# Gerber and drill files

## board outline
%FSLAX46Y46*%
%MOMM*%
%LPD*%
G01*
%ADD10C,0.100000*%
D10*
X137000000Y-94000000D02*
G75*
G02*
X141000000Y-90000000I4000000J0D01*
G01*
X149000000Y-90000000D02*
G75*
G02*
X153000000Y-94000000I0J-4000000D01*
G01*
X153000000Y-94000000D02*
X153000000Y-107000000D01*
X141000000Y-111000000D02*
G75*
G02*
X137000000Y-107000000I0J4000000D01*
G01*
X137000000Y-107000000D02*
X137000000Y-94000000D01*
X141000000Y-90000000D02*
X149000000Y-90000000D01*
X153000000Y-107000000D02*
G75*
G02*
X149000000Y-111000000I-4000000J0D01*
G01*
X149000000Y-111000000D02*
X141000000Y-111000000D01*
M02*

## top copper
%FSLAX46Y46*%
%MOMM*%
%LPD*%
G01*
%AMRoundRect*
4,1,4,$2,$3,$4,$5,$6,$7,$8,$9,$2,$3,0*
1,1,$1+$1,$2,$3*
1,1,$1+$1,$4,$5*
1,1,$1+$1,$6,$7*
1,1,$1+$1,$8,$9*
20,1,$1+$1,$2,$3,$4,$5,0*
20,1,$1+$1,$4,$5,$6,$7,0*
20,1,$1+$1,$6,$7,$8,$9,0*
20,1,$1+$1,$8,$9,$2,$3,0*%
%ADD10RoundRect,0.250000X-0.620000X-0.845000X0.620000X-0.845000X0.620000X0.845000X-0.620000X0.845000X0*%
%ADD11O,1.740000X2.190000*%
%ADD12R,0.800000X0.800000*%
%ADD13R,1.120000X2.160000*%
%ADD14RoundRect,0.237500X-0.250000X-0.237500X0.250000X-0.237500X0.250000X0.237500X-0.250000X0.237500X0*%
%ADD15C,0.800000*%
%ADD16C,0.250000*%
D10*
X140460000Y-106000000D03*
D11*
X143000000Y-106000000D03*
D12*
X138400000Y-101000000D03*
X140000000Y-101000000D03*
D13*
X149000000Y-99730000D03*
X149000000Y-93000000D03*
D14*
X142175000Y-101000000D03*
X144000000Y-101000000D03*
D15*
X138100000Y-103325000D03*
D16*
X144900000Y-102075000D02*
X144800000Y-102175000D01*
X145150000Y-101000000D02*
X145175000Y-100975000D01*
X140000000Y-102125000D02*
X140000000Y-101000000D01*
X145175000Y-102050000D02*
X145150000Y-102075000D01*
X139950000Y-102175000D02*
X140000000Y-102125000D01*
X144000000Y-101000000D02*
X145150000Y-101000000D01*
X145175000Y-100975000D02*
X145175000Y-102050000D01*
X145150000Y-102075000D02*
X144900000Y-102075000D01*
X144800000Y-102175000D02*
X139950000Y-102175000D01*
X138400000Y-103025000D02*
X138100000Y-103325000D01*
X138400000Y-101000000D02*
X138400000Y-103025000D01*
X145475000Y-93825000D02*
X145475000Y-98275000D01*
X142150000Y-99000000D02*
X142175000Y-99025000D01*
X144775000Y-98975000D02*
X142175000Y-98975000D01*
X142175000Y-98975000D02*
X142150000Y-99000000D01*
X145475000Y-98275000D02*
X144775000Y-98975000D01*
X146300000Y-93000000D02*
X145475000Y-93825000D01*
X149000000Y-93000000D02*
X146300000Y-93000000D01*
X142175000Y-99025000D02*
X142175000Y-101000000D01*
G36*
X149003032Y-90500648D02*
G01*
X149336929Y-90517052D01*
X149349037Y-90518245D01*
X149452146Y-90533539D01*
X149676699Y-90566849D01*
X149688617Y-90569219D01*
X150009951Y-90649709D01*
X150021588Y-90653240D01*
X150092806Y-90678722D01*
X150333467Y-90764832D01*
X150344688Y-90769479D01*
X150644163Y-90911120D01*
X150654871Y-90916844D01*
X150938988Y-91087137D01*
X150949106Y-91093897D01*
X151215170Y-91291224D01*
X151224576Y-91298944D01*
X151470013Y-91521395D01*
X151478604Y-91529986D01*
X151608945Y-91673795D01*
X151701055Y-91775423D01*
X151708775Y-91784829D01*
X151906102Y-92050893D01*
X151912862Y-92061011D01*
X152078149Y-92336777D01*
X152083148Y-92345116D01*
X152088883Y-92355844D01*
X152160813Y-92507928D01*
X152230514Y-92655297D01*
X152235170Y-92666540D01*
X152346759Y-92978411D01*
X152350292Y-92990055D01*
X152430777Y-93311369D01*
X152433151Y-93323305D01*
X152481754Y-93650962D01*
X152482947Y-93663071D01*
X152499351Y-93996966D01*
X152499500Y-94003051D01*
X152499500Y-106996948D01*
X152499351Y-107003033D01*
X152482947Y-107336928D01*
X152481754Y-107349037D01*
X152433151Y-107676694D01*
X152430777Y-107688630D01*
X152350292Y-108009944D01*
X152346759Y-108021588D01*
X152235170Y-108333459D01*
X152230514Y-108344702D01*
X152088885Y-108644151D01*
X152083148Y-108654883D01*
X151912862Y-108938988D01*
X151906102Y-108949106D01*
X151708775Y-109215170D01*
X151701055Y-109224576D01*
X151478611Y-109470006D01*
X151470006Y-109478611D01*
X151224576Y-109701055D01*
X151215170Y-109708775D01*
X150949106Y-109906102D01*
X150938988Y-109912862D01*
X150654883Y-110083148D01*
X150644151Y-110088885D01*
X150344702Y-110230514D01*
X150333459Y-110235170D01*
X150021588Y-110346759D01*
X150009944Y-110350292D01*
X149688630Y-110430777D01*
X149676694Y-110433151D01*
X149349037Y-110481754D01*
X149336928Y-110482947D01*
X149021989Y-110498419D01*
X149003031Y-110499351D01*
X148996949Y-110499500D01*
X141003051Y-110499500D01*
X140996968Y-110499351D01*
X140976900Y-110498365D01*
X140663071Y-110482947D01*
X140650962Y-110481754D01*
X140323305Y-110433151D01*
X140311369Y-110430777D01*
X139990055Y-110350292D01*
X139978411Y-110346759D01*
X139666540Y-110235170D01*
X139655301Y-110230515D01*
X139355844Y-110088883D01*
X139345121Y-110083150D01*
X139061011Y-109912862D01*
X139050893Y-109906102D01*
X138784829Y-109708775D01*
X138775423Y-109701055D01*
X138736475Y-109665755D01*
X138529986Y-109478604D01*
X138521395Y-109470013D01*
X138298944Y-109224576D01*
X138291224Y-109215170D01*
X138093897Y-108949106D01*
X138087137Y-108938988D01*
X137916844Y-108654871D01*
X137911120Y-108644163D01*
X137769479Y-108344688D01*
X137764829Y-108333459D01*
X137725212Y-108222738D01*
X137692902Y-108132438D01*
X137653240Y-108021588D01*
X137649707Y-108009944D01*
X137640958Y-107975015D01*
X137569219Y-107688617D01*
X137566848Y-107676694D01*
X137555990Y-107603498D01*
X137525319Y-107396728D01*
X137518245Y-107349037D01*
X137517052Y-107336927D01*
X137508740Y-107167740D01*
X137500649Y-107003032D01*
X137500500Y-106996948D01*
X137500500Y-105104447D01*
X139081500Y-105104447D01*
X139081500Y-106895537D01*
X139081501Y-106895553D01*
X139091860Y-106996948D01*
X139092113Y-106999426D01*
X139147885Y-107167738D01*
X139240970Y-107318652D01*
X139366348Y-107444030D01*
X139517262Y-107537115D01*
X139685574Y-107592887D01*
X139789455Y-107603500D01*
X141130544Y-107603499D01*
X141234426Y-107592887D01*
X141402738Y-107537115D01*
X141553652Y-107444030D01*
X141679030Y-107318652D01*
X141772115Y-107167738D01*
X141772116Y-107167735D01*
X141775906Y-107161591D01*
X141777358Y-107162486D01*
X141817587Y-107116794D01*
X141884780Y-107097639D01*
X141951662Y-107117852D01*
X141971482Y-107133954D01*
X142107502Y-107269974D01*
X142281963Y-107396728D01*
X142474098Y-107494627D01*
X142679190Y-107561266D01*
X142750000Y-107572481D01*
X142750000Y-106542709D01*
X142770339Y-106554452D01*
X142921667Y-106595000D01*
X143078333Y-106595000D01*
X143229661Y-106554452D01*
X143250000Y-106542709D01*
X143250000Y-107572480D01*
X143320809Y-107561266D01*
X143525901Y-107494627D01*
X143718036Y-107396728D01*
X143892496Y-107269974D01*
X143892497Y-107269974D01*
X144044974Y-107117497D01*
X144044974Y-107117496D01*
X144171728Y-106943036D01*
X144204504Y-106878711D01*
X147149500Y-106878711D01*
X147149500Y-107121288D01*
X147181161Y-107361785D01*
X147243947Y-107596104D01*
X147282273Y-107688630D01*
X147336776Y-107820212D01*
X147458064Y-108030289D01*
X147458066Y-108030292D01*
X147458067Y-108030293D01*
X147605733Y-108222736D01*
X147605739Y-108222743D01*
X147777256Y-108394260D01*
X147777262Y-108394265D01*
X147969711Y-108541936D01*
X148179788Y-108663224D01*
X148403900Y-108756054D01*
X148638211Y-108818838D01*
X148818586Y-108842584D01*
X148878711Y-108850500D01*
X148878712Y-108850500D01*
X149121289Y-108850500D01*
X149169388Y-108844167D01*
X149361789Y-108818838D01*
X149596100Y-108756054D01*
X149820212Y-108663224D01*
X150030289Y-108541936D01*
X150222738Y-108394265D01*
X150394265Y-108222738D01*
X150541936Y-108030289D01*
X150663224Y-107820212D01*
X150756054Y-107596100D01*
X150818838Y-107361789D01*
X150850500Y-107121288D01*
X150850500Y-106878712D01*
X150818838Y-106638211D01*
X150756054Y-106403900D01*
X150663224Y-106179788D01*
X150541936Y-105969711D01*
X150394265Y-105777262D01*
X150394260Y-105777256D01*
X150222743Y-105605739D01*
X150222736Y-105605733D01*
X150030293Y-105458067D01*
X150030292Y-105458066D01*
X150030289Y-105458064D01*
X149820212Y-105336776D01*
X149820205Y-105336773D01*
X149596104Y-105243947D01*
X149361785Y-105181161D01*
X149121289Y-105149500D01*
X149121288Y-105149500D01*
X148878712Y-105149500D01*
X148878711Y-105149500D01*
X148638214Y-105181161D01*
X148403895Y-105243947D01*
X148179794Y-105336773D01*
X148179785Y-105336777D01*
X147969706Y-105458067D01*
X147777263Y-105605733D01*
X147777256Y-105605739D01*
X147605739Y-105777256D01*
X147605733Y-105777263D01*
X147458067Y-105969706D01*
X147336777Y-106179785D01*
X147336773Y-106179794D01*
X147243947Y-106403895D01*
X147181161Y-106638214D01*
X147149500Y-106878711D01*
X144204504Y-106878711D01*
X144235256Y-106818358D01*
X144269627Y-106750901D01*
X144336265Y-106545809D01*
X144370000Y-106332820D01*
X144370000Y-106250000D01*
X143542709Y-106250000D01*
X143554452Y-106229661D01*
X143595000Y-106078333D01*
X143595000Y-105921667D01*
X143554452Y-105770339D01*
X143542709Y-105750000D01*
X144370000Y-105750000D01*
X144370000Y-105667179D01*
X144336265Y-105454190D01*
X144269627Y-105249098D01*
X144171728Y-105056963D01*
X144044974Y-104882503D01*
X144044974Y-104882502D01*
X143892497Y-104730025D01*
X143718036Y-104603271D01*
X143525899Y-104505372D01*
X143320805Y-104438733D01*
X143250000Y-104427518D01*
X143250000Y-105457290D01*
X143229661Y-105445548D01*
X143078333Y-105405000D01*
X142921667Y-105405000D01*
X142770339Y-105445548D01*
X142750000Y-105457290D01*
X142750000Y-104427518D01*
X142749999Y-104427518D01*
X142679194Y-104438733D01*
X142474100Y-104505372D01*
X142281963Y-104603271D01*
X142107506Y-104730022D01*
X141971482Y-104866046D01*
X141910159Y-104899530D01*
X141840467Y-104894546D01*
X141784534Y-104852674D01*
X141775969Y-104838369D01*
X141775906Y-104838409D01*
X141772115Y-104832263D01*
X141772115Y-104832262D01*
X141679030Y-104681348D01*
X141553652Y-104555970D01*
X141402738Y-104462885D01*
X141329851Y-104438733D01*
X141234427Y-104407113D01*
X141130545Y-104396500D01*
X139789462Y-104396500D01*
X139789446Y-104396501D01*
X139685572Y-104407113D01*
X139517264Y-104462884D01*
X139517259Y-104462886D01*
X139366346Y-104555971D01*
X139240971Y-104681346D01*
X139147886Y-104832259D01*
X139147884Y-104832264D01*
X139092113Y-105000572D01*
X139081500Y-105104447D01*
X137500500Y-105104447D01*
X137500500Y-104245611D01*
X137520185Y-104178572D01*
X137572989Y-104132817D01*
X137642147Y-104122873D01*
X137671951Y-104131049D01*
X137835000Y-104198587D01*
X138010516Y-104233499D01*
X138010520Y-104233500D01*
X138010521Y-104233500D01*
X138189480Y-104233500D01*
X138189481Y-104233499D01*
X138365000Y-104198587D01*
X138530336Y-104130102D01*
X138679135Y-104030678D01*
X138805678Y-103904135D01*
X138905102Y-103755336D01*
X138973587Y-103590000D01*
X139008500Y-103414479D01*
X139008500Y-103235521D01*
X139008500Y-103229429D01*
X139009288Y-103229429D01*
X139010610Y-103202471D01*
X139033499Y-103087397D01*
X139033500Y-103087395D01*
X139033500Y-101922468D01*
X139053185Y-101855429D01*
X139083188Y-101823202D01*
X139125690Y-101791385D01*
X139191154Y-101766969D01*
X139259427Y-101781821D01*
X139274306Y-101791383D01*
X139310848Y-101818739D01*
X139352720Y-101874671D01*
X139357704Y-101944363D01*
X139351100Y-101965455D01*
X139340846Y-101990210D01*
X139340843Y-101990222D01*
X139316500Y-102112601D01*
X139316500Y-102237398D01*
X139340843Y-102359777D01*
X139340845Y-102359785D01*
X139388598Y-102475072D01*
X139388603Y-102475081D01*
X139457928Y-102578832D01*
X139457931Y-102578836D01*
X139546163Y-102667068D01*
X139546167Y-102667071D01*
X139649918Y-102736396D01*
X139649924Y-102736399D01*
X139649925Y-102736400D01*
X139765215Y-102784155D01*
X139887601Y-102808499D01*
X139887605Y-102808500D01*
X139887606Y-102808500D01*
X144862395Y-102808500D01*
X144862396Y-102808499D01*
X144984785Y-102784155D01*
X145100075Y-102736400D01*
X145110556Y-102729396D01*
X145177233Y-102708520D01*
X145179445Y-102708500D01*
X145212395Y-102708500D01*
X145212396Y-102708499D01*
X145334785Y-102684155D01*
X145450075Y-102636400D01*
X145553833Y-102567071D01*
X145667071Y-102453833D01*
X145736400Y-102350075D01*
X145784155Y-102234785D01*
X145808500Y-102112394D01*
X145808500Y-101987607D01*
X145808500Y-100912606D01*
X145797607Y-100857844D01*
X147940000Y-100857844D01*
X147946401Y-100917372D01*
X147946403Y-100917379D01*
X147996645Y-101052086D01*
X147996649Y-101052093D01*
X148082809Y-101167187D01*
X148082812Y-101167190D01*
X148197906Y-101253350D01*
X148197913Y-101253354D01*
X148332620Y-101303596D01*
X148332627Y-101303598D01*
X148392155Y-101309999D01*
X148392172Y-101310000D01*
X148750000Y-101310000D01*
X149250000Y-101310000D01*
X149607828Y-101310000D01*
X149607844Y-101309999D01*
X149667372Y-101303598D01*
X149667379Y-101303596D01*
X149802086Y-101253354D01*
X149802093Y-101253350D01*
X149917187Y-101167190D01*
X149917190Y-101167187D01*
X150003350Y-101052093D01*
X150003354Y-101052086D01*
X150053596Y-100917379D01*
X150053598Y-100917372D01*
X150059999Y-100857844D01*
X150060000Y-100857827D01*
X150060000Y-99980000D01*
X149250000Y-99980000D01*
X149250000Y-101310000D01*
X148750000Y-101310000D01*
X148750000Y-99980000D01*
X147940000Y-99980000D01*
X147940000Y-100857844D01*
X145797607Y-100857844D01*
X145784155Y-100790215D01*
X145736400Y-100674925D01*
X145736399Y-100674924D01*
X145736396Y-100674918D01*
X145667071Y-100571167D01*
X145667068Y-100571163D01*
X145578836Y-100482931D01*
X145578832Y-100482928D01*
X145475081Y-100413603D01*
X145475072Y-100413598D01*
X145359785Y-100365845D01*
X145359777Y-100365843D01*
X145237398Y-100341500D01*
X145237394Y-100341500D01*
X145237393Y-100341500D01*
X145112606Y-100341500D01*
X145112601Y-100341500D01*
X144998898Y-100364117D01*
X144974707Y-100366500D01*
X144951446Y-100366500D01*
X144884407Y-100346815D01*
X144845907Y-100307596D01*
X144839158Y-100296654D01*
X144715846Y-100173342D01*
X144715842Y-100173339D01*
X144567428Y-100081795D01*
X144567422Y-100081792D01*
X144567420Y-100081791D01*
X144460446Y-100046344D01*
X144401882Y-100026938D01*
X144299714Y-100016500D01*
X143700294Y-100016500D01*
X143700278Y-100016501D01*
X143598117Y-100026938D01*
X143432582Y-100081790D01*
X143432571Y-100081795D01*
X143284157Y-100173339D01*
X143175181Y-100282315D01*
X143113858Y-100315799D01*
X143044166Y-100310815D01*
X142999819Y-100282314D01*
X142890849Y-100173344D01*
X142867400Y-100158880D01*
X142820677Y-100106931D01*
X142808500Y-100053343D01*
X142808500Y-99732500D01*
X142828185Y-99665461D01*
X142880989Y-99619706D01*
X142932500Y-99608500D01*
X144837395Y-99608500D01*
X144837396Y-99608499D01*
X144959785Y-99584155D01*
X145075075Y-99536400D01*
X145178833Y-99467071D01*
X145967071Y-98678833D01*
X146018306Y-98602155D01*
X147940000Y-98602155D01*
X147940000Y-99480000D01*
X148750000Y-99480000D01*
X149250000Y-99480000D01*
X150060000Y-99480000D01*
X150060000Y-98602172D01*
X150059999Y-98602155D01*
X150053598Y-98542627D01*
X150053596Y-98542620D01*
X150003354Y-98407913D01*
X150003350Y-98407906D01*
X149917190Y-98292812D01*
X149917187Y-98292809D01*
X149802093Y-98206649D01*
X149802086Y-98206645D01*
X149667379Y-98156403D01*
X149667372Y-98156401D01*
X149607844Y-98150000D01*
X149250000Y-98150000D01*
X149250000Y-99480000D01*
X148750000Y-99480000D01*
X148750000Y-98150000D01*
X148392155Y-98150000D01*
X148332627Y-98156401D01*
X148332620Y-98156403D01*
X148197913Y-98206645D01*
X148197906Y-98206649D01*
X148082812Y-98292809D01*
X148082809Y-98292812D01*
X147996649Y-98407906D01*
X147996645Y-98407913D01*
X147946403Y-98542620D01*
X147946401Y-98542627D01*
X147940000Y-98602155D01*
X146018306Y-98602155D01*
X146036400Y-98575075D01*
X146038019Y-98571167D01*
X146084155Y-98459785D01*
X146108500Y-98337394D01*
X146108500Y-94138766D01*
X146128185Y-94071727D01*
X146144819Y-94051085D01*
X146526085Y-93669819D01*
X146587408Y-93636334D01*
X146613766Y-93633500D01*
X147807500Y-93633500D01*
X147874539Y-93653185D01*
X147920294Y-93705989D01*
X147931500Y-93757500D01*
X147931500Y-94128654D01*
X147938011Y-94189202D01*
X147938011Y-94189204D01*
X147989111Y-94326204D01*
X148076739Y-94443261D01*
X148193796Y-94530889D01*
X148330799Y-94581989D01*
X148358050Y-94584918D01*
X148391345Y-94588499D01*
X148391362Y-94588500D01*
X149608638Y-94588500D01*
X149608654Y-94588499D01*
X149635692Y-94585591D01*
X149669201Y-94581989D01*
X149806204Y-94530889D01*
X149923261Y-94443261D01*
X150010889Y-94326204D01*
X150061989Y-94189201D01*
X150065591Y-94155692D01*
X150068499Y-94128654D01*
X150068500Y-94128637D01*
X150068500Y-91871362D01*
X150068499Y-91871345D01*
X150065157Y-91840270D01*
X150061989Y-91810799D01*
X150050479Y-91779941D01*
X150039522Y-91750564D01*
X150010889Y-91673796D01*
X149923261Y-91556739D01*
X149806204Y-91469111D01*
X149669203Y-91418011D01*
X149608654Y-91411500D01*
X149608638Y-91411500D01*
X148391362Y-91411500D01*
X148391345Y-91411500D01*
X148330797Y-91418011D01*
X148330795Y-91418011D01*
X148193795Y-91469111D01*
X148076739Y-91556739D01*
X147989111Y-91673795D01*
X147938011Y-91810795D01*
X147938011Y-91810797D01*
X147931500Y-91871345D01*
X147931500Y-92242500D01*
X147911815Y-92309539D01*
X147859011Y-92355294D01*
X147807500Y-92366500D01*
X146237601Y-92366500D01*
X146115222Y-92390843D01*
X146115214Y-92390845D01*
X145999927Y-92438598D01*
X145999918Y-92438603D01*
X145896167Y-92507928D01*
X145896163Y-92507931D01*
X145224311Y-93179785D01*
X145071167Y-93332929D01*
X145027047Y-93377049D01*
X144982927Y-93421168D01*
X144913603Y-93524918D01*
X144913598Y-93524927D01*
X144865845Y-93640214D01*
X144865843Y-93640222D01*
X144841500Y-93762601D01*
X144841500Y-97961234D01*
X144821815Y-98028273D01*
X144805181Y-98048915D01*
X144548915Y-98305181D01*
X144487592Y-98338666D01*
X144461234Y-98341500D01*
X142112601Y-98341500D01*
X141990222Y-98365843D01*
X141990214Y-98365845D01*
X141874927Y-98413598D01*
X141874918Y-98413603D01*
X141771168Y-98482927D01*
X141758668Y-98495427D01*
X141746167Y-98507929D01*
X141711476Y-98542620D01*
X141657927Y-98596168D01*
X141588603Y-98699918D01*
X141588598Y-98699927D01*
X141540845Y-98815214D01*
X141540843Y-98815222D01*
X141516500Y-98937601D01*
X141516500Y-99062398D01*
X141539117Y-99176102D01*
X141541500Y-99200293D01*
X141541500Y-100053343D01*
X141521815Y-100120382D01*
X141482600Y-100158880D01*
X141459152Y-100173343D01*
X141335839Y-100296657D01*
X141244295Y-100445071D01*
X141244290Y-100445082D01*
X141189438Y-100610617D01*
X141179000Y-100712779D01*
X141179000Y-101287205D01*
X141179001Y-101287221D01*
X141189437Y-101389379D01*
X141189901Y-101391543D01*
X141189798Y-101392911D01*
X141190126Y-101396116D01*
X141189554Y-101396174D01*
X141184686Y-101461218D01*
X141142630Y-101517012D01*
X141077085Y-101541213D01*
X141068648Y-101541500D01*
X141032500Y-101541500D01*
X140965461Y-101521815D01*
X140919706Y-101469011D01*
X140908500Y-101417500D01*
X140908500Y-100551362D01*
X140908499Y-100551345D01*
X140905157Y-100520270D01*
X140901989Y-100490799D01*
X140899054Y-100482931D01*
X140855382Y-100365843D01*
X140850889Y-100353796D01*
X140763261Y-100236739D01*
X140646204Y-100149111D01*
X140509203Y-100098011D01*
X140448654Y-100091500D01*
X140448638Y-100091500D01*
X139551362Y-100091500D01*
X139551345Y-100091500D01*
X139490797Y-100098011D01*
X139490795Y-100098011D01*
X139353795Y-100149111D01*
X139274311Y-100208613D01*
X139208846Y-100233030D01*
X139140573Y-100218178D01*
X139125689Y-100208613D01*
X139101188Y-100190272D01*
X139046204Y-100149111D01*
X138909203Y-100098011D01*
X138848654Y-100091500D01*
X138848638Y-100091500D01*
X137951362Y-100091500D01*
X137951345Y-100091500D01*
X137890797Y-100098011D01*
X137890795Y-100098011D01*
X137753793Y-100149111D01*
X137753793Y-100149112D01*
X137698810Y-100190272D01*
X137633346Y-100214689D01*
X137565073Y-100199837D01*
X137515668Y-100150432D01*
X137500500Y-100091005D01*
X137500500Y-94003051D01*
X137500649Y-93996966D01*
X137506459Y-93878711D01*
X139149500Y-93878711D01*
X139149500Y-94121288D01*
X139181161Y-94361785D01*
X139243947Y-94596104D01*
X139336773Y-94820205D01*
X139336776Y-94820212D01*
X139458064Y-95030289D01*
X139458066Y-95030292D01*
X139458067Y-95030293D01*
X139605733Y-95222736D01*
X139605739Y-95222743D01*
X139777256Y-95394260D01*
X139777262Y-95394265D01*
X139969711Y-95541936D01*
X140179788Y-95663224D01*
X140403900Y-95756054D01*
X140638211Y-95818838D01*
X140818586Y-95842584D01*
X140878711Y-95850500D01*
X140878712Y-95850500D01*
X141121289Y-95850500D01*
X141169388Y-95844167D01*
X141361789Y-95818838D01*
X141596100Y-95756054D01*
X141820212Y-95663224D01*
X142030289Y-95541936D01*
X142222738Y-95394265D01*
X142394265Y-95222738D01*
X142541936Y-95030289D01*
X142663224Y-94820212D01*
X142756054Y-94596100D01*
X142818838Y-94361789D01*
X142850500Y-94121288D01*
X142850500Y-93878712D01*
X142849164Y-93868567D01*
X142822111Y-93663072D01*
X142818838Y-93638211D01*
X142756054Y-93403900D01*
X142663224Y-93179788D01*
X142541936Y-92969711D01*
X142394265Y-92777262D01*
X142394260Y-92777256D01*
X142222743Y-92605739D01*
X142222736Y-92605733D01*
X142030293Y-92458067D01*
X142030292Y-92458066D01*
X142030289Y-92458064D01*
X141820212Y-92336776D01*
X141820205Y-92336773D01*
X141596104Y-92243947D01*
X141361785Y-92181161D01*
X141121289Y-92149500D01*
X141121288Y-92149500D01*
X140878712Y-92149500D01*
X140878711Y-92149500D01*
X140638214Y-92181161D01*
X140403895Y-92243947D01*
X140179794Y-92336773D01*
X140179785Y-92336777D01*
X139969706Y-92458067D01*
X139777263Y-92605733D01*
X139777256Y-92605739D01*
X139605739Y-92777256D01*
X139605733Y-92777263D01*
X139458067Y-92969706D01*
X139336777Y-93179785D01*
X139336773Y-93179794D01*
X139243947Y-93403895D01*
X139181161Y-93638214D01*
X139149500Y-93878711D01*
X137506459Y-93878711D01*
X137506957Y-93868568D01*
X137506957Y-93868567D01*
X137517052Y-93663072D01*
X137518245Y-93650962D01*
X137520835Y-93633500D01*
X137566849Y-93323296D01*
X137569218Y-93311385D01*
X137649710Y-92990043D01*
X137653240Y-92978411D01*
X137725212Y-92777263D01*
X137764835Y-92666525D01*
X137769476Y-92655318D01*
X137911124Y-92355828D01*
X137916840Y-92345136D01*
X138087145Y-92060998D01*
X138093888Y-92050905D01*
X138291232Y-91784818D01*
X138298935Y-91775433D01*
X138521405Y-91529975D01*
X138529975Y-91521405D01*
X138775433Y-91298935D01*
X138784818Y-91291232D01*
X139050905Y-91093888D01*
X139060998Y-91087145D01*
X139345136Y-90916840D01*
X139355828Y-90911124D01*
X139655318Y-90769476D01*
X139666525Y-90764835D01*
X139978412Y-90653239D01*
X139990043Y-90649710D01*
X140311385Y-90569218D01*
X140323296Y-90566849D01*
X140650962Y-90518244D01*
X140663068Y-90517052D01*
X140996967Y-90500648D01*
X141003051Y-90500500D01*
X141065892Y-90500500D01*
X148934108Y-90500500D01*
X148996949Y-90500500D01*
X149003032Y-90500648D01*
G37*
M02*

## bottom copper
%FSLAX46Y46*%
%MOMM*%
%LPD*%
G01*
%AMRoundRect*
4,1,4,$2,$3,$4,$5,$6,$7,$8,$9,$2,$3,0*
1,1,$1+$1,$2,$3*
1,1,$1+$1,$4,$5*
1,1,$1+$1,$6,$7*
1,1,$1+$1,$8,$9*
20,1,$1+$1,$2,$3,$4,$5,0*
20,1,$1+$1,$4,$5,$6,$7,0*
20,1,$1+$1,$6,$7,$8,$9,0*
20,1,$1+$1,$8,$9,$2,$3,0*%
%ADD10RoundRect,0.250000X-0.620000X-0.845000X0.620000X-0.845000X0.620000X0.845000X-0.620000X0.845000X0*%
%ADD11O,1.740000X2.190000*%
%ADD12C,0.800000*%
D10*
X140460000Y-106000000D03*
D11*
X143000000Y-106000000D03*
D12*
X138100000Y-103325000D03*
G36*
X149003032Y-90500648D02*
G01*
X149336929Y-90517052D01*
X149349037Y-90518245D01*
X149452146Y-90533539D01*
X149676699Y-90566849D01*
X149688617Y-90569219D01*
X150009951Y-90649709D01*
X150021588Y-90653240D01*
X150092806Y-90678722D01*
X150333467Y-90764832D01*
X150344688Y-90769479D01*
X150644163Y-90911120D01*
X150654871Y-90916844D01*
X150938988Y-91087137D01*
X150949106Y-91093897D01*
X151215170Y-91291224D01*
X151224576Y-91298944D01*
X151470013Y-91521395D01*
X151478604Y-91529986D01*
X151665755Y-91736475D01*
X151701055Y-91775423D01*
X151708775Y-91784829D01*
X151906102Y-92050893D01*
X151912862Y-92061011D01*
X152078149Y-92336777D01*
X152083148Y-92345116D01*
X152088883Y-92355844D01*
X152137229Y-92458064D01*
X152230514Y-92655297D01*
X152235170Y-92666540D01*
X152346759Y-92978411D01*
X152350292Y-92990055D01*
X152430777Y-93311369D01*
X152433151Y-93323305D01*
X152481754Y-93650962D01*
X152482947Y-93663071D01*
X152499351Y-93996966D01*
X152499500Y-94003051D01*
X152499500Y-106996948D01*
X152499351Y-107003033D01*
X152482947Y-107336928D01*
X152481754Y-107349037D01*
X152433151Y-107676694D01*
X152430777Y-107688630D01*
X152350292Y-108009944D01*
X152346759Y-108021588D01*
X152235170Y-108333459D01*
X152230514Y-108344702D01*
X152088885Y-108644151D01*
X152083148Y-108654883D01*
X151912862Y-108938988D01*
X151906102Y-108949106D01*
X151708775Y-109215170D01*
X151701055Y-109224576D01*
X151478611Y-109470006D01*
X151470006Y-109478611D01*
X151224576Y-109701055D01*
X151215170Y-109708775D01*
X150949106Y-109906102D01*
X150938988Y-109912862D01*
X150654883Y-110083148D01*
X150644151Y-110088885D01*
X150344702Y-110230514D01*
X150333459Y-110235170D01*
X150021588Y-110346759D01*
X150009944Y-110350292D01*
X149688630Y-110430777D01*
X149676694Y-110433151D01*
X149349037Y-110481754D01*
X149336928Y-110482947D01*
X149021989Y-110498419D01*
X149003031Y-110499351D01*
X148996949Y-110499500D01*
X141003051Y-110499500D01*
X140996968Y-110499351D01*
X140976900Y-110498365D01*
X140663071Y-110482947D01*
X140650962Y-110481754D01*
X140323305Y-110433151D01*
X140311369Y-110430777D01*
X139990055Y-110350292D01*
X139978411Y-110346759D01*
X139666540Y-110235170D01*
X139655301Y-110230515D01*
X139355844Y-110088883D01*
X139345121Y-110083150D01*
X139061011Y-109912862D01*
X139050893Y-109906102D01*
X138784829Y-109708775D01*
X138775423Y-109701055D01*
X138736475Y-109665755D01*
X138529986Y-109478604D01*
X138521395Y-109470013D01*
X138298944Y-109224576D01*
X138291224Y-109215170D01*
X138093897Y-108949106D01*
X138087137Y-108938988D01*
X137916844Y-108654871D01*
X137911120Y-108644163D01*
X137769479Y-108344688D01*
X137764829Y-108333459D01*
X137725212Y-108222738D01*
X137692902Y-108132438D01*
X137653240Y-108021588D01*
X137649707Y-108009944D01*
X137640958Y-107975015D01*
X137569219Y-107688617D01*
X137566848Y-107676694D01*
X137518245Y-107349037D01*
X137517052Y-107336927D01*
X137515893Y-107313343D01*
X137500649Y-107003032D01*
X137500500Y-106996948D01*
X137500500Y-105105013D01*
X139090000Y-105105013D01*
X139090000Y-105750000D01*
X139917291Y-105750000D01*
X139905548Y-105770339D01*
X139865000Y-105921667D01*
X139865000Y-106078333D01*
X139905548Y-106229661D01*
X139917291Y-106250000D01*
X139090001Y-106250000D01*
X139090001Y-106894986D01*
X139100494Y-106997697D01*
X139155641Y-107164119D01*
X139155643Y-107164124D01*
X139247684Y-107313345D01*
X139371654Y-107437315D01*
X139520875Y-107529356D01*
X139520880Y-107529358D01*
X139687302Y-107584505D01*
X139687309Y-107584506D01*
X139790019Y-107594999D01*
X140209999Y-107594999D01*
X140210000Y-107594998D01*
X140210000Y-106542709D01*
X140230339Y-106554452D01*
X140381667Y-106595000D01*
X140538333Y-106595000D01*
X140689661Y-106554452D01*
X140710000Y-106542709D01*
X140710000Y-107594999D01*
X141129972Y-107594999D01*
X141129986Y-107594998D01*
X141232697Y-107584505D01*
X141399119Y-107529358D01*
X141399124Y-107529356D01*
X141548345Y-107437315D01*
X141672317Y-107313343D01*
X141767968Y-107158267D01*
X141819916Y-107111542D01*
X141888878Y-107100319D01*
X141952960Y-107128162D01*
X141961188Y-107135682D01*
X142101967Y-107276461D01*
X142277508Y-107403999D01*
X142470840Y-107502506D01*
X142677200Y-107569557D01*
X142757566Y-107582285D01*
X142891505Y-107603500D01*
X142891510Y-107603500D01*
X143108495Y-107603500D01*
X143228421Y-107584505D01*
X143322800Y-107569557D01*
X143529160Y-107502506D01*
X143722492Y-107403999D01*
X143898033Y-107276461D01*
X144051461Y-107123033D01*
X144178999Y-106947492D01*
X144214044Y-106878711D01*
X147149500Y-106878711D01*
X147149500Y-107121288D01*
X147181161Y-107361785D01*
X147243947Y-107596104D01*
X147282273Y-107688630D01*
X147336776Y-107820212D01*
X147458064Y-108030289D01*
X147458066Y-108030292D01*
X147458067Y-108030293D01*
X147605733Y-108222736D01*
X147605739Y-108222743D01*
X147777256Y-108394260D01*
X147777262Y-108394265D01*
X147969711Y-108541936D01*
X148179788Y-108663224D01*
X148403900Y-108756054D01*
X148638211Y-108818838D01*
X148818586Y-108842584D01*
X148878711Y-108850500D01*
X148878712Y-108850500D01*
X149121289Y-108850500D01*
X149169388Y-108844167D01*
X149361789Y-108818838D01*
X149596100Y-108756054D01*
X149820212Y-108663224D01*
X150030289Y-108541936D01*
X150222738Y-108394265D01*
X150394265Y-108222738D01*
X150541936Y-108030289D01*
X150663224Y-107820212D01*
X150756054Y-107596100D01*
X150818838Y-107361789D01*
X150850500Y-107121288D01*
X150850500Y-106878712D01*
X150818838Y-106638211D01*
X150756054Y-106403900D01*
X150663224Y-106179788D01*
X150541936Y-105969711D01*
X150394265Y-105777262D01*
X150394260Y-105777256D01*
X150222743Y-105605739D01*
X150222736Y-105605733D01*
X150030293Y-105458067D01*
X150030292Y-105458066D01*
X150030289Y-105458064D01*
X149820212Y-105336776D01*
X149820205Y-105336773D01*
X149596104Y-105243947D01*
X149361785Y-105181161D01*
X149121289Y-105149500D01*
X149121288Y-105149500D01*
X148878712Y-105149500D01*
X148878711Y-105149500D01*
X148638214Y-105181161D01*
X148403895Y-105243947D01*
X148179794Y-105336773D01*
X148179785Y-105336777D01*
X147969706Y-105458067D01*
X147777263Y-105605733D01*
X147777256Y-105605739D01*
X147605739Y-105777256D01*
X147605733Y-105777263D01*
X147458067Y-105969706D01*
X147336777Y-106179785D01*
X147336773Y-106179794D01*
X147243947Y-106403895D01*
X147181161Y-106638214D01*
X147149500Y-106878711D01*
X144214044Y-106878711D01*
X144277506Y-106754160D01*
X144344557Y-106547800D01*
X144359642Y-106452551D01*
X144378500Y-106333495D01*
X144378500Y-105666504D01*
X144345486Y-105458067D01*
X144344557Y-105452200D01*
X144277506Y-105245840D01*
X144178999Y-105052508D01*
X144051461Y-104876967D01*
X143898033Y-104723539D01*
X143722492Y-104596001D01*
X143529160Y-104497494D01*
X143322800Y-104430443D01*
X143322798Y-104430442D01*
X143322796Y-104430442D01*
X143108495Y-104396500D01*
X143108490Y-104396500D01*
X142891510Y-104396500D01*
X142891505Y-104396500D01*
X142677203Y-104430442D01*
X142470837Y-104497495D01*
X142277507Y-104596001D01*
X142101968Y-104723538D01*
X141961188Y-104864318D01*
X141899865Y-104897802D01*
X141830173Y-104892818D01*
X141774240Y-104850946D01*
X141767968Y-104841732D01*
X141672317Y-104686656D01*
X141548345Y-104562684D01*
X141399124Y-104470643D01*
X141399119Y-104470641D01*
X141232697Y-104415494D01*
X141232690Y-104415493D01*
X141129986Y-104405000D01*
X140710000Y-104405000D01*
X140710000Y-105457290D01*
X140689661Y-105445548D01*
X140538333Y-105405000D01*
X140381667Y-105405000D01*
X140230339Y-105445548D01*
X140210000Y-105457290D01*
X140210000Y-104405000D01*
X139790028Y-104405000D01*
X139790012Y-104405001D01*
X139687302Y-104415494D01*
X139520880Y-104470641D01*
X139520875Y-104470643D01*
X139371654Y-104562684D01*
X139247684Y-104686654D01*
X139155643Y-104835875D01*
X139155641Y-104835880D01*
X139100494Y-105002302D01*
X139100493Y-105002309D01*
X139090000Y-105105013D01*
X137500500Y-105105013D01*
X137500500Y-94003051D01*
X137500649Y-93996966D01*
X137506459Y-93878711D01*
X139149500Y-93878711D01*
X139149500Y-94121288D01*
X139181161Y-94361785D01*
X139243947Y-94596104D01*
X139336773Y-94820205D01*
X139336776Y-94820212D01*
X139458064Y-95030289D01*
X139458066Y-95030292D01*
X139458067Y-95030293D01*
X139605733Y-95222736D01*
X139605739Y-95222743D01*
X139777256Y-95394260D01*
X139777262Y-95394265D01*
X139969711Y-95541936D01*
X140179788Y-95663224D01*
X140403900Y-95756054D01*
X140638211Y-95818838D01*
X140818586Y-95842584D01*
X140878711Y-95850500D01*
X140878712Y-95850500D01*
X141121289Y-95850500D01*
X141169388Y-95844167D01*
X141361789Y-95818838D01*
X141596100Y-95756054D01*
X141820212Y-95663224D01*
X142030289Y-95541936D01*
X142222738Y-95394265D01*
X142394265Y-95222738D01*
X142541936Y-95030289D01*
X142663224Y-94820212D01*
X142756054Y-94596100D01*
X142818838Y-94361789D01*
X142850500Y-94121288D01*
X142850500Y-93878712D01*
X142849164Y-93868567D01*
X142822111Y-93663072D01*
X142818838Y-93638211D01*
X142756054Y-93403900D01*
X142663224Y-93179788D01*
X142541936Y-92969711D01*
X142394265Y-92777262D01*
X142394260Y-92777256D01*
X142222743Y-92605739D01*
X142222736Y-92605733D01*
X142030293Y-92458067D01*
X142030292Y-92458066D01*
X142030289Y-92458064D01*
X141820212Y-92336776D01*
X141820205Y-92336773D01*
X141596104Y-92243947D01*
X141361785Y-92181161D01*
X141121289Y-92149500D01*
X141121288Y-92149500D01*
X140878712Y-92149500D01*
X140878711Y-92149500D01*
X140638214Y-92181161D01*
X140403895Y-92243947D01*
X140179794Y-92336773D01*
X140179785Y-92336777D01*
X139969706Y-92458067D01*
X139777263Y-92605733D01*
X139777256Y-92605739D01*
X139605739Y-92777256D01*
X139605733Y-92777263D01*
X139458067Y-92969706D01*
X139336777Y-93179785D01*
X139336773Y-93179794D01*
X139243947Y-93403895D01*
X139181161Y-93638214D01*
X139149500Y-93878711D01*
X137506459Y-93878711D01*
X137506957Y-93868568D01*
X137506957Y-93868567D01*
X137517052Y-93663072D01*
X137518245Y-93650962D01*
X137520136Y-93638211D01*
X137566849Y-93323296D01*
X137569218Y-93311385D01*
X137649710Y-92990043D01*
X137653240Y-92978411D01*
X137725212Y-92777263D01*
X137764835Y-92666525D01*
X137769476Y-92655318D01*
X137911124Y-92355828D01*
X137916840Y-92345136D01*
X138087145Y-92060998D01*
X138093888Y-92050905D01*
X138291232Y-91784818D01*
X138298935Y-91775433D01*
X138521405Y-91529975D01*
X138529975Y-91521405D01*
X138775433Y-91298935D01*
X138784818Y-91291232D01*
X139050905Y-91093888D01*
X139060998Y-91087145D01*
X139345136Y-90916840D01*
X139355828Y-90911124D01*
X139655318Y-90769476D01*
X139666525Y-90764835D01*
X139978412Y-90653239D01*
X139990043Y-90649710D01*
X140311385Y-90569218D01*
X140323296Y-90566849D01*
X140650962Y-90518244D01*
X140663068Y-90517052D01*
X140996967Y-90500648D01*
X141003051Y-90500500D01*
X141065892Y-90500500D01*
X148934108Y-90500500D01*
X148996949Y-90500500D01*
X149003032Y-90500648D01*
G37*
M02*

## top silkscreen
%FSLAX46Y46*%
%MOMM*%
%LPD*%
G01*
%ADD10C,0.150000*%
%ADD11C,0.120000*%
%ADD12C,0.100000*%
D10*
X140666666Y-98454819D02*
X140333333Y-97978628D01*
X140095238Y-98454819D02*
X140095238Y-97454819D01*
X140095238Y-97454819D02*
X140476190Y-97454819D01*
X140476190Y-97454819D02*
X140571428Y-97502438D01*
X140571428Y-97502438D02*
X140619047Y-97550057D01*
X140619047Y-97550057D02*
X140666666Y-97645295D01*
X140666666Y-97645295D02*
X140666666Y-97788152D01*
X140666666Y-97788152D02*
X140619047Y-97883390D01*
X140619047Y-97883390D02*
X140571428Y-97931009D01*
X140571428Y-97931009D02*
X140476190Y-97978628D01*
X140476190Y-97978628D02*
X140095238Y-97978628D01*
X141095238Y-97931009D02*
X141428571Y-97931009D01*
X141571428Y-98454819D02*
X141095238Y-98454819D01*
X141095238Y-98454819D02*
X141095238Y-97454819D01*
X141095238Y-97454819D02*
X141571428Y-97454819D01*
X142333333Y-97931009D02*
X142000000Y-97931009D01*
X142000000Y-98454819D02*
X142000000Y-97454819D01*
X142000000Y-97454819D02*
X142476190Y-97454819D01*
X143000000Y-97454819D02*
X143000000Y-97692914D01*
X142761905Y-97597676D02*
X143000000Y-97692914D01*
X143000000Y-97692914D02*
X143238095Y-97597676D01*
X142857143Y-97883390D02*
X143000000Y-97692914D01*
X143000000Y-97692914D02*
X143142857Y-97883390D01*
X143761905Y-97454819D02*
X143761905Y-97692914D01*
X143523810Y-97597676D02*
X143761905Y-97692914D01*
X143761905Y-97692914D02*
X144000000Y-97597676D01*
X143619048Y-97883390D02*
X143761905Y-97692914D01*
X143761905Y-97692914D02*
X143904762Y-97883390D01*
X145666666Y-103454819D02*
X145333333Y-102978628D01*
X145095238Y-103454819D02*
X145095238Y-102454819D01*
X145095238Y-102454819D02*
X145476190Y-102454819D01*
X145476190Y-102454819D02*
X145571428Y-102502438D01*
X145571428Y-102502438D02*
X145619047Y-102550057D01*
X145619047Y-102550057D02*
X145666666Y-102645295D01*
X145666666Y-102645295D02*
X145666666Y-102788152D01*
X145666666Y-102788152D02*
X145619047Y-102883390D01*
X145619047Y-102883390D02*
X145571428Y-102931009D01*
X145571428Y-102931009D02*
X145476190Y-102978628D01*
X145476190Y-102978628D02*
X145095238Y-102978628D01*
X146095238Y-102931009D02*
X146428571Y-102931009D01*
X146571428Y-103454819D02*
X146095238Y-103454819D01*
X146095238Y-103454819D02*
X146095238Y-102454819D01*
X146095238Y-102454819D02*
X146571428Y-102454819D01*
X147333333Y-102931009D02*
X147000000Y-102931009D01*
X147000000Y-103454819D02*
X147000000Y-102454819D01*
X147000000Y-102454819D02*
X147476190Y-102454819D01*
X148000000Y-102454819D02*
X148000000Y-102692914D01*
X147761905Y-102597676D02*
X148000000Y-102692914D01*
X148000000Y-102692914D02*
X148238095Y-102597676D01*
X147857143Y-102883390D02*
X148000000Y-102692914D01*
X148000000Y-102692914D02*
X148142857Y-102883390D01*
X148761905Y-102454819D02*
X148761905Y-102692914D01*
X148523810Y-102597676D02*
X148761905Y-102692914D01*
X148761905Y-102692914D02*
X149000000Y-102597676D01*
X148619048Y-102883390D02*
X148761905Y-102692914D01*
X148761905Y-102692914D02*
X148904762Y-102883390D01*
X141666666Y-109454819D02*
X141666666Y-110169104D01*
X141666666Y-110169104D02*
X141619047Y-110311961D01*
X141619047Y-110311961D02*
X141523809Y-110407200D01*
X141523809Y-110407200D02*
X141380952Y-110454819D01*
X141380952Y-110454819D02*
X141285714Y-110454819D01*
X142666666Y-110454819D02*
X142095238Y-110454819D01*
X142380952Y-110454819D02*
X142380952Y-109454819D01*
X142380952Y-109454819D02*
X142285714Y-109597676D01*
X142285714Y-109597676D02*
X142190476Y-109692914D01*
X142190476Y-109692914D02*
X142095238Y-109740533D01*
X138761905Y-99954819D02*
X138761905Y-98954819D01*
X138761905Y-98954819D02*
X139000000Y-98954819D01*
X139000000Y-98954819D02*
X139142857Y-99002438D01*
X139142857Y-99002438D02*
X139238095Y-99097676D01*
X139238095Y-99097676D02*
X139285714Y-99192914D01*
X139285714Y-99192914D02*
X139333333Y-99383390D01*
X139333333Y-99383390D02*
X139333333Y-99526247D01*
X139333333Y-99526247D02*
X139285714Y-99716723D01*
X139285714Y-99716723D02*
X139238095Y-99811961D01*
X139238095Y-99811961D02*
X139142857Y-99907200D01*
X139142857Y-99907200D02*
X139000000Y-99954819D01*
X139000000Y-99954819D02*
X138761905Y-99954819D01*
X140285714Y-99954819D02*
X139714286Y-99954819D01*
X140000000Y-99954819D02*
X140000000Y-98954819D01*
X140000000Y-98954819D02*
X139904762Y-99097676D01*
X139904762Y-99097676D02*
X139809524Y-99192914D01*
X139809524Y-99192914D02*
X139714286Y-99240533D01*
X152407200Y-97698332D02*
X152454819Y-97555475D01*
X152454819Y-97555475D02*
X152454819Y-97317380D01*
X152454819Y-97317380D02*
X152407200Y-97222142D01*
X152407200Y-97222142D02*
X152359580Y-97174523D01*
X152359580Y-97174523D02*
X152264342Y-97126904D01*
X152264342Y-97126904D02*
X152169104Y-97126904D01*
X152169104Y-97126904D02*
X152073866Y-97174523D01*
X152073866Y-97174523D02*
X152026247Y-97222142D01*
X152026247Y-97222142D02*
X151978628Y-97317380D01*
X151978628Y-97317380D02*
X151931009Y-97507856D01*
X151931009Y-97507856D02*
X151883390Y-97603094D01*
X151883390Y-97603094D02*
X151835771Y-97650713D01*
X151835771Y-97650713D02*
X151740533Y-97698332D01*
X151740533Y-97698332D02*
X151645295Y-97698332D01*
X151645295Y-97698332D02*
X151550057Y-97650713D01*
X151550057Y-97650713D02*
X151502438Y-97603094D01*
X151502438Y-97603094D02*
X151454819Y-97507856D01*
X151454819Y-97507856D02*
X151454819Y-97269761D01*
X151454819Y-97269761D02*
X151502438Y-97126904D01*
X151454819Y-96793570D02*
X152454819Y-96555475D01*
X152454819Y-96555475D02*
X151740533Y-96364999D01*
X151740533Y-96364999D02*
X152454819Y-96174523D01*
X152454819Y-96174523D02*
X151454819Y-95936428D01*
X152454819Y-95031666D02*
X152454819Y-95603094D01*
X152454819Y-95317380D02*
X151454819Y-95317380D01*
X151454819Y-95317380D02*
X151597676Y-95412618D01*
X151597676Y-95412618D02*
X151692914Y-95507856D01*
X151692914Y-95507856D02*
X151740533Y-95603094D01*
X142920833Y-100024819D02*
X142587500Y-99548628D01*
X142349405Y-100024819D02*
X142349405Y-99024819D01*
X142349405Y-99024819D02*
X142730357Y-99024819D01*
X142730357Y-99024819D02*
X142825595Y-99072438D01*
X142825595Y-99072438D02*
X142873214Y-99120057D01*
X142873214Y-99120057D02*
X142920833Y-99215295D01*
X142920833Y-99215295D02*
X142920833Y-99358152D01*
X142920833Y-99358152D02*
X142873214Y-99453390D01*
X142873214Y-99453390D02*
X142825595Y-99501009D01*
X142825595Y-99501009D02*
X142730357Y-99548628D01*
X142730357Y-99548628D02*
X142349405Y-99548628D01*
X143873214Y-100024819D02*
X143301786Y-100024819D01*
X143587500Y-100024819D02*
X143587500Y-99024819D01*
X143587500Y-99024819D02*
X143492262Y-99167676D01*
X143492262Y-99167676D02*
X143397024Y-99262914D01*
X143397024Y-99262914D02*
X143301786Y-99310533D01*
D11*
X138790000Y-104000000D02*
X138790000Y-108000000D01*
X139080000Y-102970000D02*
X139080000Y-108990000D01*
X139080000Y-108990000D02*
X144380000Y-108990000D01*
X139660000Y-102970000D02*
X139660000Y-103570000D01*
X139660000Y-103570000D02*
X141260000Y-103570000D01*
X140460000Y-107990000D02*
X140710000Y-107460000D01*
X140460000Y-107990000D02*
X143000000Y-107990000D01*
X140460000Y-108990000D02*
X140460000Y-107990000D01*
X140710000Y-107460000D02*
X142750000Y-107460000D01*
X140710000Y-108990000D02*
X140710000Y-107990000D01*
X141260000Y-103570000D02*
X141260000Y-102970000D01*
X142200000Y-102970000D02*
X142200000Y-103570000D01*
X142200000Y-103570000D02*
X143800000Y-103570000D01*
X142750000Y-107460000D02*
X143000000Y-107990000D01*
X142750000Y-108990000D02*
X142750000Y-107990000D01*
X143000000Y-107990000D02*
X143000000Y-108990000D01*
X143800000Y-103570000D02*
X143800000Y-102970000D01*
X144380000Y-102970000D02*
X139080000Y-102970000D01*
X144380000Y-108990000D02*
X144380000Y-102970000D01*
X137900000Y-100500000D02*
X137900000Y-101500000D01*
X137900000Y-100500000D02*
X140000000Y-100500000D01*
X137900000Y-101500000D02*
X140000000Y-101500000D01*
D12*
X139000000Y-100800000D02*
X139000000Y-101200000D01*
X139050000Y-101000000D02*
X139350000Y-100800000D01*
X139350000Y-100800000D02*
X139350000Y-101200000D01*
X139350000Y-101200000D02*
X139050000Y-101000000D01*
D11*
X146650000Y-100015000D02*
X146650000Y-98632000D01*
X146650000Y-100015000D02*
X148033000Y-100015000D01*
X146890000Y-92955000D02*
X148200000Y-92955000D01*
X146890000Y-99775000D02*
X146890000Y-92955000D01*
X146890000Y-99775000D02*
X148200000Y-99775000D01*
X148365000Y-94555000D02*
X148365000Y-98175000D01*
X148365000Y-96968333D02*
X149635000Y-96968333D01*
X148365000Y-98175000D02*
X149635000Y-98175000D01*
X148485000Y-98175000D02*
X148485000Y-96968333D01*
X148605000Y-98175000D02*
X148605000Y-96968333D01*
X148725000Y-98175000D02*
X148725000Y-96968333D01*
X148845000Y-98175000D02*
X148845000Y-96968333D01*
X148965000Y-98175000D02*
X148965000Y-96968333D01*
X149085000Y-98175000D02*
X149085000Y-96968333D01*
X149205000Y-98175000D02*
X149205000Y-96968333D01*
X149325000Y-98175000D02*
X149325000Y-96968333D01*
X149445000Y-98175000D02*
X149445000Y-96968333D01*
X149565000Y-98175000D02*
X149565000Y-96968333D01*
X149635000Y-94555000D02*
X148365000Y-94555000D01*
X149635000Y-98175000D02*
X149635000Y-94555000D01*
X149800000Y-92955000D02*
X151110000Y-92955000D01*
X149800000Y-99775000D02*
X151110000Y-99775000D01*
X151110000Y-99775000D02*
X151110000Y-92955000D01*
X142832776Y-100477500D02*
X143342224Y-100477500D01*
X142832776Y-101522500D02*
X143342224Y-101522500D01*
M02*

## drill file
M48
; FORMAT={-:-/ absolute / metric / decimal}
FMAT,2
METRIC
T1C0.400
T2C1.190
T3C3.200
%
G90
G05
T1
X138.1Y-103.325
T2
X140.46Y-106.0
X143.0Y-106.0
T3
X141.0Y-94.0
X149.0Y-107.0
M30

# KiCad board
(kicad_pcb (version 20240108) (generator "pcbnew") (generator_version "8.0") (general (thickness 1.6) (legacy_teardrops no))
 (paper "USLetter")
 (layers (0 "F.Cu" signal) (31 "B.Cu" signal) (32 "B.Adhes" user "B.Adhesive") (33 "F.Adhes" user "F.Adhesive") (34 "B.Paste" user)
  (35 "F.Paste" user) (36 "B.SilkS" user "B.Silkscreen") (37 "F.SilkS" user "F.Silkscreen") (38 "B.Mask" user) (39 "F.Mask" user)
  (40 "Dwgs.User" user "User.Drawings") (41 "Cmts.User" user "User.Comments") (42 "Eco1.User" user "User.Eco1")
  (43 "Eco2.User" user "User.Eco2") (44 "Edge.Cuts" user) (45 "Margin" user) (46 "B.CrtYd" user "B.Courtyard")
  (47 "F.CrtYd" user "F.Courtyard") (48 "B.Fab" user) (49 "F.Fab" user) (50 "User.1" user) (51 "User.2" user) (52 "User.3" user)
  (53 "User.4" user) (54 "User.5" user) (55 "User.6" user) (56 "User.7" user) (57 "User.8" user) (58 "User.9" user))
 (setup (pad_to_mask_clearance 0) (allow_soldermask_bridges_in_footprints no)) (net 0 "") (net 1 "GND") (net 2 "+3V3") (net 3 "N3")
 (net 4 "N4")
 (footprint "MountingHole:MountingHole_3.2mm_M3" (layer "F.Cu") (at 141 94)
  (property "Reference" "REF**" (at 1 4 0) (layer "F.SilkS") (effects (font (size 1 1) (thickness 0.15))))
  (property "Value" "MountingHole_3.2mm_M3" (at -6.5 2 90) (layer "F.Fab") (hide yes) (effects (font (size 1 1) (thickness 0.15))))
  (pad "" np_thru_hole circle (at 0 0) (size 3.2 3.2) (drill 3.2) (layers "*.Cu" "*.Mask")))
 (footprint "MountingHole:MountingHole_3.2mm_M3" (layer "F.Cu") (at 149 107)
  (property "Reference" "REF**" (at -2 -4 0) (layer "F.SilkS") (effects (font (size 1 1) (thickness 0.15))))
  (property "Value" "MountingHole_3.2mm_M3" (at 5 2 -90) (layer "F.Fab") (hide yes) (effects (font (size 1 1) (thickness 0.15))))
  (pad "" np_thru_hole circle (at 0 0) (size 3.2 3.2) (drill 3.2) (layers "F&B.Cu" "*.Mask")))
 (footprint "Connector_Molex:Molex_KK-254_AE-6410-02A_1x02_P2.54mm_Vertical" (layer "F.Cu") (at 140.46 106)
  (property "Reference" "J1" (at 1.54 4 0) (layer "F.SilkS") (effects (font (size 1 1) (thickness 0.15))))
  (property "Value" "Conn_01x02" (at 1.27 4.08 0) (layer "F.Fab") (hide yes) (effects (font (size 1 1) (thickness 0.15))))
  (fp_line (start -1.67 -2) (end -1.67 2) (stroke (width 0.12) (type solid)) (layer "F.SilkS"))
  (fp_line (start -1.38 -3.03) (end -1.38 2.99) (stroke (width 0.12) (type solid)) (layer "F.SilkS"))
  (fp_line (start -1.38 2.99) (end 3.92 2.99) (stroke (width 0.12) (type solid)) (layer "F.SilkS"))
  (fp_line (start -0.8 -3.03) (end -0.8 -2.43) (stroke (width 0.12) (type solid)) (layer "F.SilkS"))
  (fp_line (start -0.8 -2.43) (end 0.8 -2.43) (stroke (width 0.12) (type solid)) (layer "F.SilkS"))
  (fp_line (start 0 1.99) (end 0.25 1.46) (stroke (width 0.12) (type solid)) (layer "F.SilkS"))
  (fp_line (start 0 1.99) (end 2.54 1.99) (stroke (width 0.12) (type solid)) (layer "F.SilkS"))
  (fp_line (start 0 2.99) (end 0 1.99) (stroke (width 0.12) (type solid)) (layer "F.SilkS"))
  (fp_line (start 0.25 1.46) (end 2.29 1.46) (stroke (width 0.12) (type solid)) (layer "F.SilkS"))
  (fp_line (start 0.25 2.99) (end 0.25 1.99) (stroke (width 0.12) (type solid)) (layer "F.SilkS"))
  (fp_line (start 0.8 -2.43) (end 0.8 -3.03) (stroke (width 0.12) (type solid)) (layer "F.SilkS"))
  (fp_line (start 1.74 -3.03) (end 1.74 -2.43) (stroke (width 0.12) (type solid)) (layer "F.SilkS"))
  (fp_line (start 1.74 -2.43) (end 3.34 -2.43) (stroke (width 0.12) (type solid)) (layer "F.SilkS"))
  (fp_line (start 2.29 1.46) (end 2.54 1.99) (stroke (width 0.12) (type solid)) (layer "F.SilkS"))
  (fp_line (start 2.29 2.99) (end 2.29 1.99) (stroke (width 0.12) (type solid)) (layer "F.SilkS"))
  (fp_line (start 2.54 1.99) (end 2.54 2.99) (stroke (width 0.12) (type solid)) (layer "F.SilkS"))
  (fp_line (start 3.34 -2.43) (end 3.34 -3.03) (stroke (width 0.12) (type solid)) (layer "F.SilkS"))
  (fp_line (start 3.92 -3.03) (end -1.38 -3.03) (stroke (width 0.12) (type solid)) (layer "F.SilkS"))
  (fp_line (start 3.92 2.99) (end 3.92 -3.03) (stroke (width 0.12) (type solid)) (layer "F.SilkS"))
  (pad "1" thru_hole roundrect (at 0 0) (size 1.74 2.19) (drill 1.19) (layers "*.Cu" "*.Mask") (remove_unused_layers no)
   (roundrect_rratio 0.143678) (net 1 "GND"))
  (pad "2" thru_hole oval (at 2.54 0) (size 1.74 2.19) (drill 1.19) (layers "*.Cu" "*.Mask") (remove_unused_layers no) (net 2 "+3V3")))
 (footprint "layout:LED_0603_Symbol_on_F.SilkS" (layer "F.Cu") (at 139.2 101)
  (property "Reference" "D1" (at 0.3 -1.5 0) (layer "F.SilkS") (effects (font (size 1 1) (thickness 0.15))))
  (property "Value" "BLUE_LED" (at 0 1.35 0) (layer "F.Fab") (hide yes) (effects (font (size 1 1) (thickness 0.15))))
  (fp_line (start -1.3 -0.5) (end -1.3 0.5) (stroke (width 0.12) (type solid)) (layer "F.SilkS"))
  (fp_line (start -1.3 -0.5) (end 0.8 -0.5) (stroke (width 0.12) (type solid)) (layer "F.SilkS"))
  (fp_line (start -1.3 0.5) (end 0.8 0.5) (stroke (width 0.12) (type solid)) (layer "F.SilkS"))
  (fp_line (start -0.2 -0.2) (end -0.2 0.2) (stroke (width 0.1) (type solid)) (layer "F.SilkS"))
  (fp_line (start -0.15 0) (end 0.15 -0.2) (stroke (width 0.1) (type solid)) (layer "F.SilkS"))
  (fp_line (start 0.15 -0.2) (end 0.15 0.2) (stroke (width 0.1) (type solid)) (layer "F.SilkS"))
  (fp_line (start 0.15 0.2) (end -0.15 0) (stroke (width 0.1) (type solid)) (layer "F.SilkS"))
  (pad "1" smd rect (at -0.8 0 180) (size 0.8 0.8) (layers "F.Cu" "F.Paste" "F.Mask") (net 1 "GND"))
  (pad "2" smd rect (at 0.8 0 180) (size 0.8 0.8) (layers "F.Cu" "F.Paste" "F.Mask") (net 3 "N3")))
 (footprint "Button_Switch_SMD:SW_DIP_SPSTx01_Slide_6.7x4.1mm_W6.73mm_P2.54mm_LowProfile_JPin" (layer "F.Cu") (at 149 96.365 90)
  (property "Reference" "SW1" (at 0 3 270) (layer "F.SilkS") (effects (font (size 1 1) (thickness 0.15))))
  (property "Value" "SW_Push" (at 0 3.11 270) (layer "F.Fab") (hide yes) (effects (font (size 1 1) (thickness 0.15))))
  (fp_line (start -3.65 -2.35) (end -2.267 -2.35) (stroke (width 0.12) (type solid)) (layer "F.SilkS"))
  (fp_line (start -3.65 -2.35) (end -3.65 -0.967) (stroke (width 0.12) (type solid)) (layer "F.SilkS"))
  (fp_line (start 3.41 -2.11) (end 3.41 -0.8) (stroke (width 0.12) (type solid)) (layer "F.SilkS"))
  (fp_line (start -3.41 -2.11) (end 3.41 -2.11) (stroke (width 0.12) (type solid)) (layer "F.SilkS"))
  (fp_line (start -3.41 -2.11) (end -3.41 -0.8) (stroke (width 0.12) (type solid)) (layer "F.SilkS"))
  (fp_line (start 1.81 -0.635) (end -1.81 -0.635) (stroke (width 0.12) (type solid)) (layer "F.SilkS"))
  (fp_line (start -0.603333 -0.635) (end -0.603333 0.635) (stroke (width 0.12) (type solid)) (layer "F.SilkS"))
  (fp_line (start -1.81 -0.635) (end -1.81 0.635) (stroke (width 0.12) (type solid)) (layer "F.SilkS"))
  (fp_line (start -1.81 -0.515) (end -0.603333 -0.515) (stroke (width 0.12) (type solid)) (layer "F.SilkS"))
  (fp_line (start -1.81 -0.395) (end -0.603333 -0.395) (stroke (width 0.12) (type solid)) (layer "F.SilkS"))
  (fp_line (start -1.81 -0.275) (end -0.603333 -0.275) (stroke (width 0.12) (type solid)) (layer "F.SilkS"))
  (fp_line (start -1.81 -0.155) (end -0.603333 -0.155) (stroke (width 0.12) (type solid)) (layer "F.SilkS"))
  (fp_line (start -1.81 -0.035) (end -0.603333 -0.035) (stroke (width 0.12) (type solid)) (layer "F.SilkS"))
  (fp_line (start -1.81 0.085) (end -0.603333 0.085) (stroke (width 0.12) (type solid)) (layer "F.SilkS"))
  (fp_line (start -1.81 0.205) (end -0.603333 0.205) (stroke (width 0.12) (type solid)) (layer "F.SilkS"))
  (fp_line (start -1.81 0.325) (end -0.603333 0.325) (stroke (width 0.12) (type solid)) (layer "F.SilkS"))
  (fp_line (start -1.81 0.445) (end -0.603333 0.445) (stroke (width 0.12) (type solid)) (layer "F.SilkS"))
  (fp_line (start -1.81 0.565) (end -0.603333 0.565) (stroke (width 0.12) (type solid)) (layer "F.SilkS"))
  (fp_line (start 1.81 0.635) (end 1.81 -0.635) (stroke (width 0.12) (type solid)) (layer "F.SilkS"))
  (fp_line (start -1.81 0.635) (end 1.81 0.635) (stroke (width 0.12) (type solid)) (layer "F.SilkS"))
  (fp_line (start 3.41 0.8) (end 3.41 2.11) (stroke (width 0.12) (type solid)) (layer "F.SilkS"))
  (fp_line (start -3.41 0.8) (end -3.41 2.11) (stroke (width 0.12) (type solid)) (layer "F.SilkS"))
  (fp_line (start -3.41 2.11) (end 3.41 2.11) (stroke (width 0.12) (type solid)) (layer "F.SilkS"))
  (pad "1" smd rect (at -3.365 0 90) (size 2.16 1.12) (layers "F.Cu" "F.Paste" "F.Mask") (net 2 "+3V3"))
  (pad "2" smd rect (at 3.365 0 90) (size 2.16 1.12) (layers "F.Cu" "F.Paste" "F.Mask") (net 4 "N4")))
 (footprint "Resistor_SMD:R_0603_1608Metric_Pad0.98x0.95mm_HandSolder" (layer "F.Cu") (at 143.0875 101)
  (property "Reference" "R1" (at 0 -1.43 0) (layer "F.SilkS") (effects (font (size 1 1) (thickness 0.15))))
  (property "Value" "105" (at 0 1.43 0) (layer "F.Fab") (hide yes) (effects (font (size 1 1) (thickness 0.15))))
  (fp_line (start -0.254724 -0.5225) (end 0.254724 -0.5225) (stroke (width 0.12) (type solid)) (layer "F.SilkS"))
  (fp_line (start -0.254724 0.5225) (end 0.254724 0.5225) (stroke (width 0.12) (type solid)) (layer "F.SilkS"))
  (pad "1" smd roundrect (at -0.9125 0) (size 0.975 0.95) (layers "F.Cu" "F.Paste" "F.Mask") (roundrect_rratio 0.25) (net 4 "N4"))
  (pad "2" smd roundrect (at 0.9125 0) (size 0.975 0.95) (layers "F.Cu" "F.Paste" "F.Mask") (roundrect_rratio 0.25) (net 3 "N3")))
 (gr_arc (start 137 94) (mid 138.171573 91.171573) (end 141 90) (stroke (width 0.1) (type default)) (layer "Edge.Cuts"))
 (gr_arc (start 149 90) (mid 151.828427 91.171573) (end 153 94) (stroke (width 0.1) (type default)) (layer "Edge.Cuts"))
 (gr_line (start 153 94) (end 153 107) (stroke (width 0.1) (type default)) (layer "Edge.Cuts"))
 (gr_arc (start 141 111) (mid 138.171573 109.828427) (end 137 107) (stroke (width 0.1) (type default)) (layer "Edge.Cuts"))
 (gr_line (start 137 107) (end 137 94) (stroke (width 0.1) (type default)) (layer "Edge.Cuts"))
 (gr_line (start 141 90) (end 149 90) (stroke (width 0.1) (type default)) (layer "Edge.Cuts"))
 (gr_arc (start 153 107) (mid 151.828427 109.828427) (end 149 111) (stroke (width 0.1) (type default)) (layer "Edge.Cuts"))
 (gr_line (start 149 111) (end 141 111) (stroke (width 0.1) (type default)) (layer "Edge.Cuts"))
 (segment (start 144.9 102.075) (end 144.8 102.175) (width 0.25) (layer "F.Cu") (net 3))
 (segment (start 145.15 101) (end 145.175 100.975) (width 0.25) (layer "F.Cu") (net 3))
 (segment (start 140 102.125) (end 140 101) (width 0.25) (layer "F.Cu") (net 3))
 (segment (start 145.175 102.05) (end 145.15 102.075) (width 0.25) (layer "F.Cu") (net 3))
 (segment (start 139.95 102.175) (end 140 102.125) (width 0.25) (layer "F.Cu") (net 3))
 (segment (start 144 101) (end 145.15 101) (width 0.25) (layer "F.Cu") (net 3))
 (segment (start 145.175 100.975) (end 145.175 102.05) (width 0.25) (layer "F.Cu") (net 3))
 (segment (start 145.15 102.075) (end 144.9 102.075) (width 0.25) (layer "F.Cu") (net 3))
 (segment (start 144.8 102.175) (end 139.95 102.175) (width 0.25) (layer "F.Cu") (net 3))
 (segment (start 138.4 103.025) (end 138.1 103.325) (width 0.25) (layer "F.Cu") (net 1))
 (segment (start 138.4 101) (end 138.4 103.025) (width 0.25) (layer "F.Cu") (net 1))
 (via (at 138.1 103.325) (size 0.8) (drill 0.4) (layers "F.Cu" "B.Cu") (free yes) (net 1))
 (segment (start 145.475 93.825) (end 145.475 98.275) (width 0.25) (layer "F.Cu") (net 4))
 (segment (start 142.15 99) (end 142.175 99.025) (width 0.25) (layer "F.Cu") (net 4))
 (segment (start 144.775 98.975) (end 142.175 98.975) (width 0.25) (layer "F.Cu") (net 4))
 (segment (start 142.175 98.975) (end 142.15 99) (width 0.25) (layer "F.Cu") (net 4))
 (segment (start 145.475 98.275) (end 144.775 98.975) (width 0.25) (layer "F.Cu") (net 4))
 (segment (start 146.3 93) (end 145.475 93.825) (width 0.25) (layer "F.Cu") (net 4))
 (segment (start 149 93) (end 146.3 93) (width 0.25) (layer "F.Cu") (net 4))
 (segment (start 142.175 99.025) (end 142.175 101) (width 0.25) (layer "F.Cu") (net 4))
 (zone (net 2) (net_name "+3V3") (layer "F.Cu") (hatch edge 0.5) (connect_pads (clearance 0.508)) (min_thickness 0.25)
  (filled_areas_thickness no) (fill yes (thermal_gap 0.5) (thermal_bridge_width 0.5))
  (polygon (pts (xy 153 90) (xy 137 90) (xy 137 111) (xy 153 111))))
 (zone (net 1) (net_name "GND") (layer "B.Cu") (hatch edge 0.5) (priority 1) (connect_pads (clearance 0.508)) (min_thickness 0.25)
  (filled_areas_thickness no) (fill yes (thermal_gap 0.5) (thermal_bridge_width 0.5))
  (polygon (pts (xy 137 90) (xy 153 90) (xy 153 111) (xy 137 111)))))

